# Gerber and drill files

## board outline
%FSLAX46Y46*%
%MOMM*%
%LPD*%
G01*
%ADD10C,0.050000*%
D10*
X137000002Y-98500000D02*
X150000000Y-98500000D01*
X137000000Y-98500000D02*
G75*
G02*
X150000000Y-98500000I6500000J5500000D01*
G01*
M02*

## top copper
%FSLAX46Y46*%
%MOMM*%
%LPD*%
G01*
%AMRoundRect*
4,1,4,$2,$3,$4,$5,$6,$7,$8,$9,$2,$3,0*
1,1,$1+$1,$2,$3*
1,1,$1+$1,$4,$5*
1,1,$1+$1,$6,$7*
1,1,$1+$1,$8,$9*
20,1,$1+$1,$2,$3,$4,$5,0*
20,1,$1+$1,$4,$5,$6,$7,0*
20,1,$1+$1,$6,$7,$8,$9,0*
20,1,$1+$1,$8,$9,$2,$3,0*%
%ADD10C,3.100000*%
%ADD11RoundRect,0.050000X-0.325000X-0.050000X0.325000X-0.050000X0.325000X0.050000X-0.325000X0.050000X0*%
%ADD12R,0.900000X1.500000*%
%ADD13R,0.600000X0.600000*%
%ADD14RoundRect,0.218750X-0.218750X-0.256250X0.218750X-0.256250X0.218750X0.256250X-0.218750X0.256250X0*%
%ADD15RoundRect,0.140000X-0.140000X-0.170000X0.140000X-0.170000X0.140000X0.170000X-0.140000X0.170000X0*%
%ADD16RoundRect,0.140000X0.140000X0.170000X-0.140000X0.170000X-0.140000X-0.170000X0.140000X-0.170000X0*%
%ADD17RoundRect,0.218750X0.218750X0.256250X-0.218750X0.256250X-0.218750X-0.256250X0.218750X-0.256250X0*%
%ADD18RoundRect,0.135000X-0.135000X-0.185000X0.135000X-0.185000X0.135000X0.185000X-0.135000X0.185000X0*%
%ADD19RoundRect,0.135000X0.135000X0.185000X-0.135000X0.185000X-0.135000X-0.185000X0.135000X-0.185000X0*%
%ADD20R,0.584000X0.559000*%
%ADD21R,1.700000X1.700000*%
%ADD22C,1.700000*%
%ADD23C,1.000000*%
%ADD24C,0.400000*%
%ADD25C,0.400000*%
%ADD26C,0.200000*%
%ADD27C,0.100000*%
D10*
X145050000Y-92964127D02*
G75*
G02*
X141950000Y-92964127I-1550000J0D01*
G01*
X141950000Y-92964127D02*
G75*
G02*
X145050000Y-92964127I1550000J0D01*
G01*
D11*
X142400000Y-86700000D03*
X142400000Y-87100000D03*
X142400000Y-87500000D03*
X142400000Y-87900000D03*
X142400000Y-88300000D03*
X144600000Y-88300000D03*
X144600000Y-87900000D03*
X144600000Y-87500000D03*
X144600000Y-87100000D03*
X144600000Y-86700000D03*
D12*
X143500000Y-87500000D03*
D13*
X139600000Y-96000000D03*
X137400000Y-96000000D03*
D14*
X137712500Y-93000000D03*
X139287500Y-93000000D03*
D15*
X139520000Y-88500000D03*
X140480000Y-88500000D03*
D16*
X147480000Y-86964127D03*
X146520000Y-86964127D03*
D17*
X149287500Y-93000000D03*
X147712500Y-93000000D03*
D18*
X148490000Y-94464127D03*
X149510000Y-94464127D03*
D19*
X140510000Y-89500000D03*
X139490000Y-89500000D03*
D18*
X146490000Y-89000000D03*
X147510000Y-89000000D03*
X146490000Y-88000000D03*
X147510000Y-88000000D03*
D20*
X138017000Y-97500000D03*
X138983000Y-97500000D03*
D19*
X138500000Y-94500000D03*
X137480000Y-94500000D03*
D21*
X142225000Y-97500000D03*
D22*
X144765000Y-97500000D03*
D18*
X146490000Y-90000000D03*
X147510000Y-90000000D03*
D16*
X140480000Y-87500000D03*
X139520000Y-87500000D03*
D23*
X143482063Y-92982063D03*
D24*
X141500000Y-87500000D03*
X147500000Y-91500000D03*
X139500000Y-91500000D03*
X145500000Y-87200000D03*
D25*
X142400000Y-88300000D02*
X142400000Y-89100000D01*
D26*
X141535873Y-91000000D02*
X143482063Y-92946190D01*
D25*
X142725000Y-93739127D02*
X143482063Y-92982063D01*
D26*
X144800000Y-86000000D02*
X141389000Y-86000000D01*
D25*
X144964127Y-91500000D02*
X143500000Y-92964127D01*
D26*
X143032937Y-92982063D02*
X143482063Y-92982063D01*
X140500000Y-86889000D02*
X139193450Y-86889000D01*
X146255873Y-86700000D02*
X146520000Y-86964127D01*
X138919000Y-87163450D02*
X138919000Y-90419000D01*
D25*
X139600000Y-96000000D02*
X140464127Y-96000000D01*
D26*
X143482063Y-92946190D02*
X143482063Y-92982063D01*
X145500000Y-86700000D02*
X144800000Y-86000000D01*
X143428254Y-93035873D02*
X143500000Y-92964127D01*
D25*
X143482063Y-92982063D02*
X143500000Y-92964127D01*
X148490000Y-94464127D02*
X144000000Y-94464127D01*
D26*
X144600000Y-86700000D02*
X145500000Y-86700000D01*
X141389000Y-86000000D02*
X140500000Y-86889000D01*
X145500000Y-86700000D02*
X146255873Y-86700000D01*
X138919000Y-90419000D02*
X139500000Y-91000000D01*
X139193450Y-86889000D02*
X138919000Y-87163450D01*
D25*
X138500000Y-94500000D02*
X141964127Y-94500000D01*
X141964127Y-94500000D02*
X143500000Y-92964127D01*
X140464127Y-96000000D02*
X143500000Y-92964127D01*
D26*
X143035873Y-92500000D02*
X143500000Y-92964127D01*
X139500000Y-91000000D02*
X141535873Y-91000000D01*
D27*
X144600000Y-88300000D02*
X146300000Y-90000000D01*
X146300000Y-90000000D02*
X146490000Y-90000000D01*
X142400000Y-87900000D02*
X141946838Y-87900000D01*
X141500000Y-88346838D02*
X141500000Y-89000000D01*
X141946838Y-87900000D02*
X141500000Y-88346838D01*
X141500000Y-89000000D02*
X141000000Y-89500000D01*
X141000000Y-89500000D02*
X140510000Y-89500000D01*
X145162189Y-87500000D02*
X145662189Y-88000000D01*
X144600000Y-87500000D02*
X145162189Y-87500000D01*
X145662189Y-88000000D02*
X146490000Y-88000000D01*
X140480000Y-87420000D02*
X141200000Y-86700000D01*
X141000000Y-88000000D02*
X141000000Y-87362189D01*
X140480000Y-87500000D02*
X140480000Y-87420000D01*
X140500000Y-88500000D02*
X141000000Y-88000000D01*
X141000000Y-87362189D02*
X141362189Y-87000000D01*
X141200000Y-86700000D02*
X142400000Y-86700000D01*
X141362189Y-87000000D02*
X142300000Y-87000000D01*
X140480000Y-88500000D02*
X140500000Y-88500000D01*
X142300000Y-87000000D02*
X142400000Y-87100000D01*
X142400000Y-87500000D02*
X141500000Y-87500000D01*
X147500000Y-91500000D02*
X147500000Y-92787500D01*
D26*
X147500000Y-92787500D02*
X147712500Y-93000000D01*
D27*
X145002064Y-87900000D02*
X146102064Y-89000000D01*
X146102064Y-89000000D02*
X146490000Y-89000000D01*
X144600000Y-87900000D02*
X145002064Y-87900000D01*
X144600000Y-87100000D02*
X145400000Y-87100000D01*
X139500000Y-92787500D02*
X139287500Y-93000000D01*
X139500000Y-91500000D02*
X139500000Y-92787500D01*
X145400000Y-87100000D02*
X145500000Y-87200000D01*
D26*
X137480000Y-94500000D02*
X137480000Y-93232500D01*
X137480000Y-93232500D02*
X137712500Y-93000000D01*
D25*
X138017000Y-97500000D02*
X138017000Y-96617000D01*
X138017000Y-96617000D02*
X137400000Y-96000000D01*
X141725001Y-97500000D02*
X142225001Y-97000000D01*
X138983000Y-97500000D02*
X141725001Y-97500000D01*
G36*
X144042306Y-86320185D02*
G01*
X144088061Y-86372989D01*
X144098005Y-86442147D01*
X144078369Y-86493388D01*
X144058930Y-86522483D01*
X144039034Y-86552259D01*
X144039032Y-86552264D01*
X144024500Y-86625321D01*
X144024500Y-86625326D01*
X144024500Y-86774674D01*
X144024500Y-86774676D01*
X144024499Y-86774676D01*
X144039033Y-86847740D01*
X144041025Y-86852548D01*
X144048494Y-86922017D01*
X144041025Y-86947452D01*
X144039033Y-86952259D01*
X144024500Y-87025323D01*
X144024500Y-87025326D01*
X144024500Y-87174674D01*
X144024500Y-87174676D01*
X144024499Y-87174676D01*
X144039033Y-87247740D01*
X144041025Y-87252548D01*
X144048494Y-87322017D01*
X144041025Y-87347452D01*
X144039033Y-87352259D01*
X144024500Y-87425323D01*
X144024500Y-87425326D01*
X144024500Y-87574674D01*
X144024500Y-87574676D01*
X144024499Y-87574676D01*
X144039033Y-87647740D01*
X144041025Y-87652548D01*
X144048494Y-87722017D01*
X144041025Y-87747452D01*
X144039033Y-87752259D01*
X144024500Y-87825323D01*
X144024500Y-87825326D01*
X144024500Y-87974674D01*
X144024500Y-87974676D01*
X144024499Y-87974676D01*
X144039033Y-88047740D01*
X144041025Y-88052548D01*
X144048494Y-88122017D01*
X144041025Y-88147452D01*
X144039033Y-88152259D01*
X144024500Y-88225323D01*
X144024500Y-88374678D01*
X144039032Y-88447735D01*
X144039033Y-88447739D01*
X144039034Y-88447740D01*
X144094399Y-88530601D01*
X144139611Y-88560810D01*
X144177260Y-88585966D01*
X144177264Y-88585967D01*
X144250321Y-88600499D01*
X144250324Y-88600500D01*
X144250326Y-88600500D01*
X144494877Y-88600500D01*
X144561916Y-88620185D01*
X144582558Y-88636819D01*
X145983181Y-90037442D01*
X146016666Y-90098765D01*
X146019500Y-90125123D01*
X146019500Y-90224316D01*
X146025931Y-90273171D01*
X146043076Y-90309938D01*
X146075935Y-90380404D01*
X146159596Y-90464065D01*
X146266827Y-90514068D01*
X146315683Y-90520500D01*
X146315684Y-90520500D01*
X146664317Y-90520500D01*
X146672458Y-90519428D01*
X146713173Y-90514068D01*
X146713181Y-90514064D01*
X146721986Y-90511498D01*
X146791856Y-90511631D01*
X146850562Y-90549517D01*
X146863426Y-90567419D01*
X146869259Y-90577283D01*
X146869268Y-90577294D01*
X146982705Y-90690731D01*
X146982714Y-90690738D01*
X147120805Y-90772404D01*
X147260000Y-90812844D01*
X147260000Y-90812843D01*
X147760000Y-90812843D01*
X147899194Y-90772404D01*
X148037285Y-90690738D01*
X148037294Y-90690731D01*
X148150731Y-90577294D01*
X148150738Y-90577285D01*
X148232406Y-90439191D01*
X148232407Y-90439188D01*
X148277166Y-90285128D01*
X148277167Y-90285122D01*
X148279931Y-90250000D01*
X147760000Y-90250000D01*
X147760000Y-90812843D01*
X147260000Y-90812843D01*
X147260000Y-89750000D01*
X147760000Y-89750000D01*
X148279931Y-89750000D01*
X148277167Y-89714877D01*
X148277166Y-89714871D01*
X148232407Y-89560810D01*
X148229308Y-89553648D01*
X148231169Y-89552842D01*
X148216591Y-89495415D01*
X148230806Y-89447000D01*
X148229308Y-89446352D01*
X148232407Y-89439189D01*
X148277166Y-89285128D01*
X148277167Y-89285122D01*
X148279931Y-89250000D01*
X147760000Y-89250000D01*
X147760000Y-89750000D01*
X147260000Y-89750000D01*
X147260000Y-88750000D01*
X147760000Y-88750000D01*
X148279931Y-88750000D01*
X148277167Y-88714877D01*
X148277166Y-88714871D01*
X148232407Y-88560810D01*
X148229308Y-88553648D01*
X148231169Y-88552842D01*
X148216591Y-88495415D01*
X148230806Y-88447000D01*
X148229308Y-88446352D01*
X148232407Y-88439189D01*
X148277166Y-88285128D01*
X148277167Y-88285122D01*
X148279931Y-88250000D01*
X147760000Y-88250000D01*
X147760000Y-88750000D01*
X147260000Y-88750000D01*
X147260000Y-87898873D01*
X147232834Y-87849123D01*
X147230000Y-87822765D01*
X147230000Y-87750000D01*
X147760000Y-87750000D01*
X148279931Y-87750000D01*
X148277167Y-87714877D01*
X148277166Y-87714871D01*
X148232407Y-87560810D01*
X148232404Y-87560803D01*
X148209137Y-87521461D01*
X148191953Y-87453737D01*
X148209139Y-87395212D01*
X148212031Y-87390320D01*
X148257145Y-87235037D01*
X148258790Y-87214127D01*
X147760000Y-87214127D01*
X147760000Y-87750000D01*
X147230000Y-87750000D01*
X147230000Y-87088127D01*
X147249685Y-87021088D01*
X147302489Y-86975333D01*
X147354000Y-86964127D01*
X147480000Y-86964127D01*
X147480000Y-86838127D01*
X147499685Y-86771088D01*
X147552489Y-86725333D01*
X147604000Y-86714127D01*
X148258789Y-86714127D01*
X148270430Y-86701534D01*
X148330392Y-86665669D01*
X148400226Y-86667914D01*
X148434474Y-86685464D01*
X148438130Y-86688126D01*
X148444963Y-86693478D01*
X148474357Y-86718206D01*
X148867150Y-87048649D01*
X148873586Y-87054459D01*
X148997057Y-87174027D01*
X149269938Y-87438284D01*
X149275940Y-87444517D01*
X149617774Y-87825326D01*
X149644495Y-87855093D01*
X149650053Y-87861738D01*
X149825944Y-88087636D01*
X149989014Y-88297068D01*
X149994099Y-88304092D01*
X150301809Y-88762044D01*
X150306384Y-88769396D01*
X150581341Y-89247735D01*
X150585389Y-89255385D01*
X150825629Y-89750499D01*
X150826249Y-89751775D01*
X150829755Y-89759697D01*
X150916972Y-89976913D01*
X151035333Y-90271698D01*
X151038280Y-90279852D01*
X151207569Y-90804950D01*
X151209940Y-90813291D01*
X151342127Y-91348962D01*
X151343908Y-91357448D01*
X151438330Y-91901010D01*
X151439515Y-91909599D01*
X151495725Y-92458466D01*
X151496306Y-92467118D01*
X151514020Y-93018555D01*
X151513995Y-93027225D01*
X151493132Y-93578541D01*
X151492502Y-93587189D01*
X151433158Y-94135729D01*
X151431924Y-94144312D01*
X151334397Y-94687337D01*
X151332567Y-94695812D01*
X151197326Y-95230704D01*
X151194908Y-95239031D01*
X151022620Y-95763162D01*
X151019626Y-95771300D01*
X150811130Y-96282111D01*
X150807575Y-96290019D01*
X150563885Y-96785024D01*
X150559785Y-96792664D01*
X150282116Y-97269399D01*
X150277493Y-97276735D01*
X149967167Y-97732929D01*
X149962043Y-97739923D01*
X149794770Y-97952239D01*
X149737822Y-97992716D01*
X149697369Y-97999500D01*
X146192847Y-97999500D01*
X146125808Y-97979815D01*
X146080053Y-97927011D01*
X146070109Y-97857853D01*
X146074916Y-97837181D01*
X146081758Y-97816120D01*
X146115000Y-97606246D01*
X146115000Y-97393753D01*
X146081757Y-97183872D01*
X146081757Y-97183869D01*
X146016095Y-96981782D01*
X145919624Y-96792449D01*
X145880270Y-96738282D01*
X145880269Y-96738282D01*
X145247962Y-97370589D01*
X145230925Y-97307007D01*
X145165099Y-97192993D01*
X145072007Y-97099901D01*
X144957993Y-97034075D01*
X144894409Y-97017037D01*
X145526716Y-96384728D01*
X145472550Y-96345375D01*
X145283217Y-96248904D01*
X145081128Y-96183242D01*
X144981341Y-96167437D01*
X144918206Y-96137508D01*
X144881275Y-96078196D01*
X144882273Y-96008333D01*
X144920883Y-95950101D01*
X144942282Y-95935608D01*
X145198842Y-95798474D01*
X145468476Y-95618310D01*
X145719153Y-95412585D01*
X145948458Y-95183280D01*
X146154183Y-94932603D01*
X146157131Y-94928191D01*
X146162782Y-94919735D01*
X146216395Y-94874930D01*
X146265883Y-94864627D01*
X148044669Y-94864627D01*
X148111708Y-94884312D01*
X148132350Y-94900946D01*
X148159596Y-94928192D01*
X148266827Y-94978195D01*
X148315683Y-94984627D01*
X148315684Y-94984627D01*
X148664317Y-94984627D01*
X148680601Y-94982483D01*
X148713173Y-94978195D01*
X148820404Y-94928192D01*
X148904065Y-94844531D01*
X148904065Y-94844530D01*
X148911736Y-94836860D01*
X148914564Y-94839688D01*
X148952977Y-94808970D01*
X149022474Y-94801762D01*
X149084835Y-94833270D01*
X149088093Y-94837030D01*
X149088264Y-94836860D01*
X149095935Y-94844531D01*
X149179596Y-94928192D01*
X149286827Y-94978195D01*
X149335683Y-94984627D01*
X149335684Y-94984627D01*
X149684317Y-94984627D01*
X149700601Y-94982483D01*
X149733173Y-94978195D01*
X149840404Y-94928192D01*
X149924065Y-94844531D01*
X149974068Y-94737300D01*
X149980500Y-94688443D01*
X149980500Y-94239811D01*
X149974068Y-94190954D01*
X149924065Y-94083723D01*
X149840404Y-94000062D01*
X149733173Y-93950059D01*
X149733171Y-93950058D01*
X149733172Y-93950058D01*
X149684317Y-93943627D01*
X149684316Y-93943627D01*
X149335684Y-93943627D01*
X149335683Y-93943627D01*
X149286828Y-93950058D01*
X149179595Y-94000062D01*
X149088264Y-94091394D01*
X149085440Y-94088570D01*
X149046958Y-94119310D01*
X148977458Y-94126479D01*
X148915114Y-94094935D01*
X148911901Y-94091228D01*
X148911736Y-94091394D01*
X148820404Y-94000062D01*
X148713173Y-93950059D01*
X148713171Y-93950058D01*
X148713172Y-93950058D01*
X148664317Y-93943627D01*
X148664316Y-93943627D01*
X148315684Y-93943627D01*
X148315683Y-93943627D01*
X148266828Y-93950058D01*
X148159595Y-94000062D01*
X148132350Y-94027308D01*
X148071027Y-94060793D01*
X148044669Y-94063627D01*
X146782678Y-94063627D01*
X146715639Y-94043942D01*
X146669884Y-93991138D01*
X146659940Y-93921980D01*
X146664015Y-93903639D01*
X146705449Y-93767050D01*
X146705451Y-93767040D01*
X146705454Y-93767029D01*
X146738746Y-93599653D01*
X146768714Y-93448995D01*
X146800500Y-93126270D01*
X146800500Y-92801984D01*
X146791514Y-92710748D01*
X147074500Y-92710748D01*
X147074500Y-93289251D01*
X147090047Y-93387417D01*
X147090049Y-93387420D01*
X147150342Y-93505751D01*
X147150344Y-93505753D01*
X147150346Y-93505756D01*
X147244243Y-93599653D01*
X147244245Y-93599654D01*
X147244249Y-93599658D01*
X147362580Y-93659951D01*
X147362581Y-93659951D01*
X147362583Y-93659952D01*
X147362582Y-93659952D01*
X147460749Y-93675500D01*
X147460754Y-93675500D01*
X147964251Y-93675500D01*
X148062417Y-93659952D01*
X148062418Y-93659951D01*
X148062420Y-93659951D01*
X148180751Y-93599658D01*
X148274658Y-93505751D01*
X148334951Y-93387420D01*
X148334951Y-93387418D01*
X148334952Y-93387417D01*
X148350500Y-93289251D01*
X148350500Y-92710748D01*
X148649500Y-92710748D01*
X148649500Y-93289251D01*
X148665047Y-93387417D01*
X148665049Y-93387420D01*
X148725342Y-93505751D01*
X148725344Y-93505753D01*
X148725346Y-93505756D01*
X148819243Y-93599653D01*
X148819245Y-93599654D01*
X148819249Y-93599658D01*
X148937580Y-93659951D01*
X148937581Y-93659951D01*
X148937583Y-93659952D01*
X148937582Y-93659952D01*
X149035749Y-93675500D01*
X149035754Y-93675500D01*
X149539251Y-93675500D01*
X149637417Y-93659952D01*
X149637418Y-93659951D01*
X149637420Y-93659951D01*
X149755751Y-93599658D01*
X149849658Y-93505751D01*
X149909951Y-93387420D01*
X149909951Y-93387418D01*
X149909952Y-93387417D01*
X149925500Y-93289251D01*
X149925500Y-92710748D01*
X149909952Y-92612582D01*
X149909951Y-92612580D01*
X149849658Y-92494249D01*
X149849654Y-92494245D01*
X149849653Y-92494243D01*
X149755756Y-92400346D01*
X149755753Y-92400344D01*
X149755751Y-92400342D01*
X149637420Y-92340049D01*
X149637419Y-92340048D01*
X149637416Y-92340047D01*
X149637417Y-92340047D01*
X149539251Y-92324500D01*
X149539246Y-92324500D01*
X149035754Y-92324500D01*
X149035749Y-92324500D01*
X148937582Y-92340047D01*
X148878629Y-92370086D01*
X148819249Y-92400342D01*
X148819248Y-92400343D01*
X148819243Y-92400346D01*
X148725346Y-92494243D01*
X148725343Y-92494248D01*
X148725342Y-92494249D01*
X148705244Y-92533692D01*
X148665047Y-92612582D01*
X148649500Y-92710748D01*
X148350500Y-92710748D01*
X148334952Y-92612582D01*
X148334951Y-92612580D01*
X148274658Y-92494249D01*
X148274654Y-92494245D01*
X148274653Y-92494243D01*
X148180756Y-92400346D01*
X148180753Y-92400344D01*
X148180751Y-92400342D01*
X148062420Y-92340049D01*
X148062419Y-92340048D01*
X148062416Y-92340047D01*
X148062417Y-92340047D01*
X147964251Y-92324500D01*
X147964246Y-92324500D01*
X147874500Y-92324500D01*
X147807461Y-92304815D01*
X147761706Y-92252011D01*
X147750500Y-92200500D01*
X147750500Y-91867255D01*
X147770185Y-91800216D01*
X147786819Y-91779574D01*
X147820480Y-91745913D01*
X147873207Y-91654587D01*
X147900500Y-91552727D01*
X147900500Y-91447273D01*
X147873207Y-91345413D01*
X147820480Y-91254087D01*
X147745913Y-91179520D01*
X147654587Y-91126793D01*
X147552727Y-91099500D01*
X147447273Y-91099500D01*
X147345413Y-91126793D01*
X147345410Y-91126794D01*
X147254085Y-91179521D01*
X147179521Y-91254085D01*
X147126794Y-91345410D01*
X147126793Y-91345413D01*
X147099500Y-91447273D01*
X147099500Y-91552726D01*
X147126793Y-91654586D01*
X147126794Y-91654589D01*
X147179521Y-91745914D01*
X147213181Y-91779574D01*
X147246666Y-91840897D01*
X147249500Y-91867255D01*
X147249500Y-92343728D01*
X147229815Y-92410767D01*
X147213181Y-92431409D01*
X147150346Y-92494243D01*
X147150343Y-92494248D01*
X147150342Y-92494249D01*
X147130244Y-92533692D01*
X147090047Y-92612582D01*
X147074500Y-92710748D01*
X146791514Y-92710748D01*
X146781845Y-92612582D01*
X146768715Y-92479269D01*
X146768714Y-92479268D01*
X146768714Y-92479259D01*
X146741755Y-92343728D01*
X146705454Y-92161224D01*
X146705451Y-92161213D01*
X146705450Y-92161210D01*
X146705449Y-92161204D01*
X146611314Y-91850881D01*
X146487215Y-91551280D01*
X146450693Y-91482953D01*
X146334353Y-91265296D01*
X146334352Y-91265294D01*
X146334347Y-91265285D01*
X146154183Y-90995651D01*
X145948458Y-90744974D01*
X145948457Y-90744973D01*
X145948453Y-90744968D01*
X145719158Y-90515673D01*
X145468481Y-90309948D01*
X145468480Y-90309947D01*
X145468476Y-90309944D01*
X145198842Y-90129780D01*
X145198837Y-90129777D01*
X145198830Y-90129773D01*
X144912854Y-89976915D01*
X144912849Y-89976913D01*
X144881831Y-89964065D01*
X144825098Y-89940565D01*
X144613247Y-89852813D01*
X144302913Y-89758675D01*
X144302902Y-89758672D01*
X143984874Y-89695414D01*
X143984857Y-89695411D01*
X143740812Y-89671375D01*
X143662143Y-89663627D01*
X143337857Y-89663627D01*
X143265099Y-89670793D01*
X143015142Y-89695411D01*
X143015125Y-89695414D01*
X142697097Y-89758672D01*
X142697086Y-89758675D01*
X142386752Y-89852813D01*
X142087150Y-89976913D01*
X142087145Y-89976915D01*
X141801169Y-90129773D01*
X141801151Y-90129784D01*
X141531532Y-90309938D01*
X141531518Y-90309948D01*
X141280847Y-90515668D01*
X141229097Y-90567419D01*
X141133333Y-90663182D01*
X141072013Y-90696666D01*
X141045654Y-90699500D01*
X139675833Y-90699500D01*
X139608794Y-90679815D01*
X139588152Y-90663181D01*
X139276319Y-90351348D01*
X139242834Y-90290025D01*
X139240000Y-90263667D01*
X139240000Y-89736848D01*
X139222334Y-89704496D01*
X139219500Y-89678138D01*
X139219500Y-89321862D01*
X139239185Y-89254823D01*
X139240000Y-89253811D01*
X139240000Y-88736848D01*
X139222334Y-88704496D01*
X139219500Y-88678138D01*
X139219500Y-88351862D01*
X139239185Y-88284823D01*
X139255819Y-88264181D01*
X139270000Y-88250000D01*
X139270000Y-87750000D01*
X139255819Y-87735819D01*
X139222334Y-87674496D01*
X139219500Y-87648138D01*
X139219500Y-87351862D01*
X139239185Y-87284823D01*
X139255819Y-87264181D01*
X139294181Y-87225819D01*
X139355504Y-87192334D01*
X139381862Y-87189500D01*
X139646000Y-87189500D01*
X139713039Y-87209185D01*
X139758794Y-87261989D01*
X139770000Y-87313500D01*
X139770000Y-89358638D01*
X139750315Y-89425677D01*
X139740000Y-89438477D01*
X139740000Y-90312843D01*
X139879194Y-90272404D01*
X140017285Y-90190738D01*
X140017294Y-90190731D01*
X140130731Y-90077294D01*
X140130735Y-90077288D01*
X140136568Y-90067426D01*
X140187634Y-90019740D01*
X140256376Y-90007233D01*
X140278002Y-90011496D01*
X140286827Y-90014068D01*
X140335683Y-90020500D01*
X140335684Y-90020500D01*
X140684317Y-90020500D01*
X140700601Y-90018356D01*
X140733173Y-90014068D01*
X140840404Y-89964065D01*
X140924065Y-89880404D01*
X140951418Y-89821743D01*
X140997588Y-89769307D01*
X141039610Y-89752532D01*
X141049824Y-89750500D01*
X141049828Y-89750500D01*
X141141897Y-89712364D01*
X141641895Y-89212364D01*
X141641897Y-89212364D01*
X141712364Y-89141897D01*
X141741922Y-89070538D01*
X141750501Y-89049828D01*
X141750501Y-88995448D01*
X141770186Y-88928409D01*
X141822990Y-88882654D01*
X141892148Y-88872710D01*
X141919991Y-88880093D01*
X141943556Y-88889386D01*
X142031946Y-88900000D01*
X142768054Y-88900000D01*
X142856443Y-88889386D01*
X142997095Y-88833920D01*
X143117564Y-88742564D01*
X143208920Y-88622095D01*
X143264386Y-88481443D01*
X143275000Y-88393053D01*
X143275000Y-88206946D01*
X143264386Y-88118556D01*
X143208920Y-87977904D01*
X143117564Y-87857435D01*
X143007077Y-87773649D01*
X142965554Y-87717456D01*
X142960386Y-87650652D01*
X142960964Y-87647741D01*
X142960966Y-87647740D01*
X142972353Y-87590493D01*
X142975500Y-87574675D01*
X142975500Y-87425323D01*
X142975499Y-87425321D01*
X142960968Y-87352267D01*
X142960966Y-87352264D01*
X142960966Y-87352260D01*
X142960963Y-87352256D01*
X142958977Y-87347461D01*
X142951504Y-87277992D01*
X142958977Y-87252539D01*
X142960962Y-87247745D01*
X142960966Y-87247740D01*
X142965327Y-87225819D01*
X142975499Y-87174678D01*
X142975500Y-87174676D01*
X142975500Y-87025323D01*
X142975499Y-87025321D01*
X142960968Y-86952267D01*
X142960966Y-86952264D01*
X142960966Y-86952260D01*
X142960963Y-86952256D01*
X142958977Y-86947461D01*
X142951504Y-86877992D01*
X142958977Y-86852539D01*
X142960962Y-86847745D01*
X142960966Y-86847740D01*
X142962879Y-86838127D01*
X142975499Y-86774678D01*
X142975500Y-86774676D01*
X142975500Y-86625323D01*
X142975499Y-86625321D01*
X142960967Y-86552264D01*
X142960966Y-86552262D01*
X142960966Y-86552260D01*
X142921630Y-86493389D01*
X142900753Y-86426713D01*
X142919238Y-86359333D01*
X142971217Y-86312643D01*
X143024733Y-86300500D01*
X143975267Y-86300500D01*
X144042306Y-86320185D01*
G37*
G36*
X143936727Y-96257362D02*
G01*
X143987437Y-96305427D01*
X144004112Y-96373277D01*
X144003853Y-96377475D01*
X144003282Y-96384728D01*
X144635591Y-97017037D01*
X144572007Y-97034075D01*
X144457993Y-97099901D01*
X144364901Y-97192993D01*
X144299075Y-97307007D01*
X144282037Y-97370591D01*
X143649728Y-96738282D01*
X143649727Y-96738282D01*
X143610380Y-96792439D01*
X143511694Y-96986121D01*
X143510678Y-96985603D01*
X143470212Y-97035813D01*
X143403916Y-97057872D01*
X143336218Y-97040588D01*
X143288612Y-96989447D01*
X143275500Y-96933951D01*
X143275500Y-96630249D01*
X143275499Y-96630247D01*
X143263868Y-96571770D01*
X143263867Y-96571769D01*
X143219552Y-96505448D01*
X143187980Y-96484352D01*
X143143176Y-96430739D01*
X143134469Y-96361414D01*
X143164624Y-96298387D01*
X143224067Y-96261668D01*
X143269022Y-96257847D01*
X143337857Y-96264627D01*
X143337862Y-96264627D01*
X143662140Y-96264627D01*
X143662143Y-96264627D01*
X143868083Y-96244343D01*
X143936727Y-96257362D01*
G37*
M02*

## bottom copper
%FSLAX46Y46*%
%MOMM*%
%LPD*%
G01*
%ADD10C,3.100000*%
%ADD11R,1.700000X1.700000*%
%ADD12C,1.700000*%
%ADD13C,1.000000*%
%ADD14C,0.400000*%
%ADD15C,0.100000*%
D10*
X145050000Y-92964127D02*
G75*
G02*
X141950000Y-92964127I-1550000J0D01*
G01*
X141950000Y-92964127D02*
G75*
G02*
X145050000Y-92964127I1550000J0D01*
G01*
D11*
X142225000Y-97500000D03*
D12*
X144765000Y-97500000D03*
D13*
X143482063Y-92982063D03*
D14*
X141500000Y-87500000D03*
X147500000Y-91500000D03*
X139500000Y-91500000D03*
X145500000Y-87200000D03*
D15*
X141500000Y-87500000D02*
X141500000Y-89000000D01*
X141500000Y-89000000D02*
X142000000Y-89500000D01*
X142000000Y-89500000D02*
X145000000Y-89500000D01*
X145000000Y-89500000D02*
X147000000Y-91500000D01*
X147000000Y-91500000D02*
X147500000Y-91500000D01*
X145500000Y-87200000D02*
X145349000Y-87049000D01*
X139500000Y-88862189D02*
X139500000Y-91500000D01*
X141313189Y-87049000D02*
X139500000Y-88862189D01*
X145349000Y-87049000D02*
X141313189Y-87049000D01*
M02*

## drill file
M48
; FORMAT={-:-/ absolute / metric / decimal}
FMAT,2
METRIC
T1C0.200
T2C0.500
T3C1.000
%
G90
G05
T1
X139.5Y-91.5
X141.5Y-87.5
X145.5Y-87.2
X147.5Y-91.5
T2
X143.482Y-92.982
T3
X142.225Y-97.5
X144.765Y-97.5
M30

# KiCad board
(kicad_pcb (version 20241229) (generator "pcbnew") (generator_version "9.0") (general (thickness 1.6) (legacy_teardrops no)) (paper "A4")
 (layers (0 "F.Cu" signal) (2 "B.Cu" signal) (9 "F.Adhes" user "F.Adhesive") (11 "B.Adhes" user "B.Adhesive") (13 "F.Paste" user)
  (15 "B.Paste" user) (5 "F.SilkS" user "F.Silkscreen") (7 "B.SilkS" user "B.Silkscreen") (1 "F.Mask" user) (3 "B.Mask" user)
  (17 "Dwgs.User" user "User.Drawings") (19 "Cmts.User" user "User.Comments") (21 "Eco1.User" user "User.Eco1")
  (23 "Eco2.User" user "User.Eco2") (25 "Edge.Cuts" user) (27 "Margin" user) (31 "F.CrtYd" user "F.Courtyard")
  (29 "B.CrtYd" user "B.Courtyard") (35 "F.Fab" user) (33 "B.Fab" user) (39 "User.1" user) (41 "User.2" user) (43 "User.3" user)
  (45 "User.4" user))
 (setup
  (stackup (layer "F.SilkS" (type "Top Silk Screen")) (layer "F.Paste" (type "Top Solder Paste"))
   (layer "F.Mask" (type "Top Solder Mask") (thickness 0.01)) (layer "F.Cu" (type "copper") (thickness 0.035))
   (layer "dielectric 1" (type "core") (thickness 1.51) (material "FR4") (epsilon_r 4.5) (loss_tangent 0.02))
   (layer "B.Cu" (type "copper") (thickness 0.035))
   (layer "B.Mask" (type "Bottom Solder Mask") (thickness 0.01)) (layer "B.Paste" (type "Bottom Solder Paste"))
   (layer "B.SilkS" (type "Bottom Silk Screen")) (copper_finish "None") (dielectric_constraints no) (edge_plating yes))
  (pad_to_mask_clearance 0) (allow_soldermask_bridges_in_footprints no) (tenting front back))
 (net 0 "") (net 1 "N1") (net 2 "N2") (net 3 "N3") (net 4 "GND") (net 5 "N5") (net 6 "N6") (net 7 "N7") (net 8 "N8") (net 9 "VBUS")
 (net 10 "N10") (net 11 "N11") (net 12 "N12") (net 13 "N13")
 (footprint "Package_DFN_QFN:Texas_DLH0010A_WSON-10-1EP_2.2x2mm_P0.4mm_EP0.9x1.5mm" (layer "F.Cu") (at 143.5 87.5)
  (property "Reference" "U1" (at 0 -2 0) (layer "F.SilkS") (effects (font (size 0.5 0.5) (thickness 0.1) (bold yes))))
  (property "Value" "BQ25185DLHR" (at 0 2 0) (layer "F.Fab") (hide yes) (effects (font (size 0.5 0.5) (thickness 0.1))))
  (pad "" smd roundrect (at 0 0) (size 0.84 1.41) (layers "F.Paste") (roundrect_rratio 0.25))
  (pad "1" smd roundrect (at -1.1 -0.8) (size 0.75 0.2) (layers "F.Cu" "F.Mask" "F.Paste") (roundrect_rratio 0.25) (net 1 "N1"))
  (pad "2" smd roundrect (at -1.1 -0.4) (size 0.75 0.2) (layers "F.Cu" "F.Mask" "F.Paste") (roundrect_rratio 0.25) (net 1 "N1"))
  (pad "3" smd roundrect (at -1.1 0) (size 0.75 0.2) (layers "F.Cu" "F.Mask" "F.Paste") (roundrect_rratio 0.25) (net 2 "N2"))
  (pad "4" smd roundrect (at -1.1 0.4) (size 0.75 0.2) (layers "F.Cu" "F.Mask" "F.Paste") (roundrect_rratio 0.25) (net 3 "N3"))
  (pad "5" smd roundrect (at -1.1 0.8) (size 0.75 0.2) (layers "F.Cu" "F.Mask" "F.Paste") (roundrect_rratio 0.25) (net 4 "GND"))
  (pad "6" smd roundrect (at 1.1 0.8) (size 0.75 0.2) (layers "F.Cu" "F.Mask" "F.Paste") (roundrect_rratio 0.25) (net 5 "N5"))
  (pad "7" smd roundrect (at 1.1 0.4) (size 0.75 0.2) (layers "F.Cu" "F.Mask" "F.Paste") (roundrect_rratio 0.25) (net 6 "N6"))
  (pad "8" smd roundrect (at 1.1 0) (size 0.75 0.2) (layers "F.Cu" "F.Mask" "F.Paste") (roundrect_rratio 0.25) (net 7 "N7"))
  (pad "9" smd roundrect (at 1.1 -0.4) (size 0.75 0.2) (layers "F.Cu" "F.Mask" "F.Paste") (roundrect_rratio 0.25) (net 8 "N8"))
  (pad "10" smd roundrect (at 1.1 -0.8) (size 0.75 0.2) (layers "F.Cu" "F.Mask" "F.Paste") (roundrect_rratio 0.25) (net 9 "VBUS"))
  (pad "11" smd rect (at 0 0) (size 0.9 1.5) (layers "F.Cu" "F.Mask") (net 4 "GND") (zone_connect 2)))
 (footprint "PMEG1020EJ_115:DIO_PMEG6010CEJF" (layer "F.Cu") (at 138.5 96 180)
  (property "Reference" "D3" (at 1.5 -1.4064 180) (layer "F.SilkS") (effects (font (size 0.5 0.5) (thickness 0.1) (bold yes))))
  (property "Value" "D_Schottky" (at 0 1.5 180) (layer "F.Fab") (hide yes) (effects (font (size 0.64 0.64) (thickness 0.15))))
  (pad "1" smd rect (at -1.1 0 180) (size 0.6 0.6) (layers "F.Cu" "F.Mask") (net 9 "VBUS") (solder_mask_margin 0.102))
  (pad "2" smd rect (at 1.1 0 180) (size 0.6 0.6) (layers "F.Cu" "F.Mask") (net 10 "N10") (solder_mask_margin 0.102)))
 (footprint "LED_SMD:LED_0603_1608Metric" (layer "F.Cu") (at 138.5 93)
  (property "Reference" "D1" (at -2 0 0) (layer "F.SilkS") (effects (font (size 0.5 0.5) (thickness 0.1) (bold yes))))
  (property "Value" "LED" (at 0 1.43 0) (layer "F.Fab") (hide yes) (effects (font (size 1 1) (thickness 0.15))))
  (pad "1" smd roundrect (at -0.7875 0) (size 0.875 0.95) (layers "F.Cu" "F.Mask" "F.Paste") (roundrect_rratio 0.25) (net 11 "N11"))
  (pad "2" smd roundrect (at 0.7875 0) (size 0.875 0.95) (layers "F.Cu" "F.Mask" "F.Paste") (roundrect_rratio 0.25) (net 8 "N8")))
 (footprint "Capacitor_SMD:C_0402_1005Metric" (layer "F.Cu") (at 140 88.5)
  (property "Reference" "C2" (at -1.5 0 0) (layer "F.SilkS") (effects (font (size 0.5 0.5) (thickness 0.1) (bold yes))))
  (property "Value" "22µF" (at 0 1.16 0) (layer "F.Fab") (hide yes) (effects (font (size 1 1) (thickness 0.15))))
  (pad "1" smd roundrect (at -0.48 0) (size 0.56 0.62) (layers "F.Cu" "F.Mask" "F.Paste") (roundrect_rratio 0.25) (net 4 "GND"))
  (pad "2" smd roundrect (at 0.48 0) (size 0.56 0.62) (layers "F.Cu" "F.Mask" "F.Paste") (roundrect_rratio 0.25) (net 1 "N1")))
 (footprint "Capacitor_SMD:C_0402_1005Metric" (layer "F.Cu") (at 147 86.964127 180)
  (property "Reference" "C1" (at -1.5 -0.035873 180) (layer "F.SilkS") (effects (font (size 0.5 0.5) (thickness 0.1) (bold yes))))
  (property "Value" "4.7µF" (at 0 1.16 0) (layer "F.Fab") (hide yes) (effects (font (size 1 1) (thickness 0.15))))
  (pad "1" smd roundrect (at -0.48 0 180) (size 0.56 0.62) (layers "F.Cu" "F.Mask" "F.Paste") (roundrect_rratio 0.25) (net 4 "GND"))
  (pad "2" smd roundrect (at 0.48 0 180) (size 0.56 0.62) (layers "F.Cu" "F.Mask" "F.Paste") (roundrect_rratio 0.25) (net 9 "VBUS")))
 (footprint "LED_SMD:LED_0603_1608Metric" (layer "F.Cu") (at 148.5 93 180)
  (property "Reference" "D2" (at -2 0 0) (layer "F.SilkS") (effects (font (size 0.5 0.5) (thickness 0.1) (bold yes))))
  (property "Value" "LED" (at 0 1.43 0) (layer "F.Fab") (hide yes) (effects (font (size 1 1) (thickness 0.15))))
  (pad "1" smd roundrect (at -0.7875 0 180) (size 0.875 0.95) (layers "F.Cu" "F.Mask" "F.Paste") (roundrect_rratio 0.25) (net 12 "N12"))
  (pad "2" smd roundrect (at 0.7875 0 180) (size 0.875 0.95) (layers "F.Cu" "F.Mask" "F.Paste") (roundrect_rratio 0.25) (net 2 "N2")))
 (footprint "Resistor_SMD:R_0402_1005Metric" (layer "F.Cu") (at 149 94.464127)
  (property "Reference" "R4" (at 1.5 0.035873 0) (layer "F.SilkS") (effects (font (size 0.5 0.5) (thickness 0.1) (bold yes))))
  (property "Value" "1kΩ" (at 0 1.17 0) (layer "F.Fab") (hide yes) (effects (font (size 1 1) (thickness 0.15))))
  (pad "1" smd roundrect (at -0.51 0) (size 0.54 0.64) (layers "F.Cu" "F.Mask" "F.Paste") (roundrect_rratio 0.25) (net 9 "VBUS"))
  (pad "2" smd roundrect (at 0.51 0) (size 0.54 0.64) (layers "F.Cu" "F.Mask" "F.Paste") (roundrect_rratio 0.25) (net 12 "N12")))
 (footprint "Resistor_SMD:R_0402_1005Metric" (layer "F.Cu") (at 140 89.5 180)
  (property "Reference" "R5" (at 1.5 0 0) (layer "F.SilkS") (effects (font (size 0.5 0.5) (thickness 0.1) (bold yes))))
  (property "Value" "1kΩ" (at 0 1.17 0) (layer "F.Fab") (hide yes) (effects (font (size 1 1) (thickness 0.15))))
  (pad "1" smd roundrect (at -0.51 0 180) (size 0.54 0.64) (layers "F.Cu" "F.Mask" "F.Paste") (roundrect_rratio 0.25) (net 3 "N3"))
  (pad "2" smd roundrect (at 0.51 0 180) (size 0.54 0.64) (layers "F.Cu" "F.Mask" "F.Paste") (roundrect_rratio 0.25) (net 4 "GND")))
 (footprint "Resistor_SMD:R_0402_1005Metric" (layer "F.Cu") (at 147 89)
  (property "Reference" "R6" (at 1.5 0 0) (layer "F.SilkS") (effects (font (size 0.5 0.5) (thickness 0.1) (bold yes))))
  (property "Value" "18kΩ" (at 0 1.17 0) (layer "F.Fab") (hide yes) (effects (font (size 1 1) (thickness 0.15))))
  (pad "1" smd roundrect (at -0.51 0) (size 0.54 0.64) (layers "F.Cu" "F.Mask" "F.Paste") (roundrect_rratio 0.25) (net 6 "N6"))
  (pad "2" smd roundrect (at 0.51 0) (size 0.54 0.64) (layers "F.Cu" "F.Mask" "F.Paste") (roundrect_rratio 0.25) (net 4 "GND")))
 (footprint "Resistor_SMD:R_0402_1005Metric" (layer "F.Cu") (at 147 88)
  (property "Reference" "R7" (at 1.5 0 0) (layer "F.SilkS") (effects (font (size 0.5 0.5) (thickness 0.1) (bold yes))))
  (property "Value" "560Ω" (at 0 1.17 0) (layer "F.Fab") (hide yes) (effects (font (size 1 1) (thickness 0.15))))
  (pad "1" smd roundrect (at -0.51 0) (size 0.54 0.64) (layers "F.Cu" "F.Mask" "F.Paste") (roundrect_rratio 0.25) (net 7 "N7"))
  (pad "2" smd roundrect (at 0.51 0) (size 0.54 0.64) (layers "F.Cu" "F.Mask" "F.Paste") (roundrect_rratio 0.25) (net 4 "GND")))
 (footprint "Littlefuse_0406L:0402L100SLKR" (layer "F.Cu") (at 138.5 97.5)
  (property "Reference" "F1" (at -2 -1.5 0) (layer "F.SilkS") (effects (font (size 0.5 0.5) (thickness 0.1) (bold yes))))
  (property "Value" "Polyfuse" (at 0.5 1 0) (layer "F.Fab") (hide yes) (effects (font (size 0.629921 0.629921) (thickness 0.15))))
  (pad "1" smd rect (at -0.483 0) (size 0.584 0.559) (layers "F.Cu" "F.Mask" "F.Paste") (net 10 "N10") (solder_mask_margin 0.102))
  (pad "2" smd rect (at 0.483 0) (size 0.584 0.559) (layers "F.Cu" "F.Mask" "F.Paste") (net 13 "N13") (solder_mask_margin 0.102)))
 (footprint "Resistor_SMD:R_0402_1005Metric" (layer "F.Cu") (at 137.99 94.5 180)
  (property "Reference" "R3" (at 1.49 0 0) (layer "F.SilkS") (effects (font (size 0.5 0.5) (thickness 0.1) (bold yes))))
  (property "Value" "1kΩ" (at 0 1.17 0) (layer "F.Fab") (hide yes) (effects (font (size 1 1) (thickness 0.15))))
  (pad "1" smd roundrect (at -0.51 0 180) (size 0.54 0.64) (layers "F.Cu" "F.Mask" "F.Paste") (roundrect_rratio 0.25) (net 9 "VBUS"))
  (pad "2" smd roundrect (at 0.51 0 180) (size 0.54 0.64) (layers "F.Cu" "F.Mask" "F.Paste") (roundrect_rratio 0.25) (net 11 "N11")))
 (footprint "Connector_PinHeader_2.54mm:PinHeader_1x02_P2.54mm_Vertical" (layer "F.Cu") (at 142.225 97.5 90)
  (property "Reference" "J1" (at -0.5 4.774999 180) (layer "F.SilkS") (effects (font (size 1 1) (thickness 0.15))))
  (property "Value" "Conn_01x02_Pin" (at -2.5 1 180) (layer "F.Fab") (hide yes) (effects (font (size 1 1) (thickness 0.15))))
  (pad "1" thru_hole rect (at 0 0 90) (size 1.7 1.7) (drill 1) (layers "*.Cu" "*.Mask") (remove_unused_layers no) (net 13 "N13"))
  (pad "2" thru_hole circle (at 0 2.54 90) (size 1.7 1.7) (drill 1) (layers "*.Cu" "*.Mask") (remove_unused_layers no) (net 4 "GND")))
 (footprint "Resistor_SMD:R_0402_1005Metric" (layer "F.Cu") (at 147 90)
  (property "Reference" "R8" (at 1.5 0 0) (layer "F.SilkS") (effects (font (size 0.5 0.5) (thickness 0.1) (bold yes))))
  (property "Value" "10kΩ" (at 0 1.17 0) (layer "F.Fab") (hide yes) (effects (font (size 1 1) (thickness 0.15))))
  (pad "1" smd roundrect (at -0.51 0) (size 0.54 0.64) (layers "F.Cu" "F.Mask" "F.Paste") (roundrect_rratio 0.25) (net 5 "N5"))
  (pad "2" smd roundrect (at 0.51 0) (size 0.54 0.64) (layers "F.Cu" "F.Mask" "F.Paste") (roundrect_rratio 0.25) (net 4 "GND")))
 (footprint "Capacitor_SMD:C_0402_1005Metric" (layer "F.Cu") (at 140 87.5 180)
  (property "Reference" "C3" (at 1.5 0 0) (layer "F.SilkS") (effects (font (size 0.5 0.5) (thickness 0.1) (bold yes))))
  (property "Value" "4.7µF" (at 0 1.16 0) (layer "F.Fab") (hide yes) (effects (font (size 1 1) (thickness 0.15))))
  (pad "1" smd roundrect (at -0.48 0 180) (size 0.56 0.62) (layers "F.Cu" "F.Mask" "F.Paste") (roundrect_rratio 0.25) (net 1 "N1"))
  (pad "2" smd roundrect (at 0.48 0 180) (size 0.56 0.62) (layers "F.Cu" "F.Mask" "F.Paste") (roundrect_rratio 0.25) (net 4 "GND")))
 (gr_circle (center 143.5 92.964127) (end 146.5 92.964127) (stroke (width 0.2) (type solid)) (fill yes) (layer "F.Cu") (net 9))
 (gr_circle (center 143.5 92.964127) (end 146.5 92.964127) (stroke (width 0.2) (type solid)) (fill yes) (layer "B.Cu") (net 9))
 (gr_line (start 137.000002 98.5) (end 150 98.5) (stroke (width 0.05) (type default)) (layer "Edge.Cuts"))
 (gr_arc (start 137 98.5) (mid 143.5 84.485307) (end 150 98.5) (stroke (width 0.05) (type default)) (layer "Edge.Cuts"))
 (segment (start 142.4 88.3) (end 142.4 89.1) (width 0.4) (layer "F.Cu") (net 4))
 (segment (start 141.535873 91) (end 143.482063 92.94619) (width 0.2) (layer "F.Cu") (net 9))
 (segment (start 142.725 93.739127) (end 143.482063 92.982063) (width 0.4) (layer "F.Cu") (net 9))
 (segment (start 144.8 86) (end 141.389 86) (width 0.2) (layer "F.Cu") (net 9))
 (segment (start 144.964127 91.5) (end 143.5 92.964127) (width 0.4) (layer "F.Cu") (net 9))
 (segment (start 143.032937 92.982063) (end 143.482063 92.982063) (width 0.2) (layer "F.Cu") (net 9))
 (segment (start 140.5 86.889) (end 139.19345 86.889) (width 0.2) (layer "F.Cu") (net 9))
 (segment (start 146.255873 86.7) (end 146.52 86.964127) (width 0.2) (layer "F.Cu") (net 9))
 (segment (start 138.919 87.16345) (end 138.919 90.419) (width 0.2) (layer "F.Cu") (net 9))
 (segment (start 139.6 96) (end 140.464127 96) (width 0.4) (layer "F.Cu") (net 9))
 (segment (start 143.482063 92.94619) (end 143.482063 92.982063) (width 0.2) (layer "F.Cu") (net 9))
 (segment (start 145.5 86.7) (end 144.8 86) (width 0.2) (layer "F.Cu") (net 9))
 (segment (start 143.428254 93.035873) (end 143.5 92.964127) (width 0.2) (layer "F.Cu") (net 9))
 (segment (start 143.482063 92.982063) (end 143.5 92.964127) (width 0.4) (layer "F.Cu") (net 9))
 (segment (start 148.49 94.464127) (end 144 94.464127) (width 0.4) (layer "F.Cu") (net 9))
 (segment (start 144.6 86.7) (end 145.5 86.7) (width 0.2) (layer "F.Cu") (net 9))
 (segment (start 141.389 86) (end 140.5 86.889) (width 0.2) (layer "F.Cu") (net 9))
 (segment (start 145.5 86.7) (end 146.255873 86.7) (width 0.2) (layer "F.Cu") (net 9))
 (segment (start 138.919 90.419) (end 139.5 91) (width 0.2) (layer "F.Cu") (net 9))
 (segment (start 139.19345 86.889) (end 138.919 87.16345) (width 0.2) (layer "F.Cu") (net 9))
 (segment (start 138.5 94.5) (end 141.964127 94.5) (width 0.4) (layer "F.Cu") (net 9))
 (segment (start 141.964127 94.5) (end 143.5 92.964127) (width 0.4) (layer "F.Cu") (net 9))
 (segment (start 140.464127 96) (end 143.5 92.964127) (width 0.4) (layer "F.Cu") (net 9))
 (segment (start 143.035873 92.5) (end 143.5 92.964127) (width 0.2) (layer "F.Cu") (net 9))
 (segment (start 139.5 91) (end 141.535873 91) (width 0.2) (layer "F.Cu") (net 9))
 (via (at 143.482063 92.982063) (size 1) (drill 0.5) (layers "F.Cu" "B.Cu") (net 9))
 (segment (start 144.6 88.3) (end 146.3 90) (width 0.1) (layer "F.Cu") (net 5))
 (segment (start 146.3 90) (end 146.49 90) (width 0.1) (layer "F.Cu") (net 5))
 (segment (start 142.4 87.9) (end 141.946838 87.9) (width 0.1) (layer "F.Cu") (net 3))
 (segment (start 141.5 88.346838) (end 141.5 89) (width 0.1) (layer "F.Cu") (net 3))
 (segment (start 141.946838 87.9) (end 141.5 88.346838) (width 0.1) (layer "F.Cu") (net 3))
 (segment (start 141.5 89) (end 141 89.5) (width 0.1) (layer "F.Cu") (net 3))
 (segment (start 141 89.5) (end 140.51 89.5) (width 0.1) (layer "F.Cu") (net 3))
 (segment (start 145.162189 87.5) (end 145.662189 88) (width 0.1) (layer "F.Cu") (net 7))
 (segment (start 144.6 87.5) (end 145.162189 87.5) (width 0.1) (layer "F.Cu") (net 7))
 (segment (start 145.662189 88) (end 146.49 88) (width 0.1) (layer "F.Cu") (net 7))
 (segment (start 140.48 87.42) (end 141.2 86.7) (width 0.1) (layer "F.Cu") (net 1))
 (segment (start 141 88) (end 141 87.362189) (width 0.1) (layer "F.Cu") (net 1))
 (segment (start 140.48 87.5) (end 140.48 87.42) (width 0.1) (layer "F.Cu") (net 1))
 (segment (start 140.5 88.5) (end 141 88) (width 0.1) (layer "F.Cu") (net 1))
 (segment (start 141 87.362189) (end 141.362189 87) (width 0.1) (layer "F.Cu") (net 1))
 (segment (start 141.2 86.7) (end 142.4 86.7) (width 0.1) (layer "F.Cu") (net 1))
 (segment (start 141.362189 87) (end 142.3 87) (width 0.1) (layer "F.Cu") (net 1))
 (segment (start 140.48 88.5) (end 140.5 88.5) (width 0.1) (layer "F.Cu") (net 1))
 (segment (start 142.3 87) (end 142.4 87.1) (width 0.1) (layer "F.Cu") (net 1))
 (segment (start 142.4 87.5) (end 141.5 87.5) (width 0.1) (layer "F.Cu") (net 2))
 (segment (start 147.5 91.5) (end 147.5 92.7875) (width 0.1) (layer "F.Cu") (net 2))
 (segment (start 147.5 92.7875) (end 147.7125 93) (width 0.2) (layer "F.Cu") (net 2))
 (via (at 141.5 87.5) (size 0.4) (drill 0.2) (layers "F.Cu" "B.Cu") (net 2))
 (via (at 147.5 91.5) (size 0.4) (drill 0.2) (layers "F.Cu" "B.Cu") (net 2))
 (segment (start 141.5 87.5) (end 141.5 89) (width 0.1) (layer "B.Cu") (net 2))
 (segment (start 141.5 89) (end 142 89.5) (width 0.1) (layer "B.Cu") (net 2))
 (segment (start 142 89.5) (end 145 89.5) (width 0.1) (layer "B.Cu") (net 2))
 (segment (start 145 89.5) (end 147 91.5) (width 0.1) (layer "B.Cu") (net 2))
 (segment (start 147 91.5) (end 147.5 91.5) (width 0.1) (layer "B.Cu") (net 2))
 (segment (start 145.002064 87.9) (end 146.102064 89) (width 0.1) (layer "F.Cu") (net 6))
 (segment (start 146.102064 89) (end 146.49 89) (width 0.1) (layer "F.Cu") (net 6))
 (segment (start 144.6 87.9) (end 145.002064 87.9) (width 0.1) (layer "F.Cu") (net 6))
 (segment (start 144.6 87.1) (end 145.4 87.1) (width 0.1) (layer "F.Cu") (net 8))
 (segment (start 139.5 92.7875) (end 139.2875 93) (width 0.1) (layer "F.Cu") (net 8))
 (segment (start 139.5 91.5) (end 139.5 92.7875) (width 0.1) (layer "F.Cu") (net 8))
 (segment (start 145.4 87.1) (end 145.5 87.2) (width 0.1) (layer "F.Cu") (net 8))
 (via (at 139.5 91.5) (size 0.4) (drill 0.2) (layers "F.Cu" "B.Cu") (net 8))
 (via (at 145.5 87.2) (size 0.4) (drill 0.2) (layers "F.Cu" "B.Cu") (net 8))
 (segment (start 145.5 87.2) (end 145.349 87.049) (width 0.1) (layer "B.Cu") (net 8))
 (segment (start 139.5 88.862189) (end 139.5 91.5) (width 0.1) (layer "B.Cu") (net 8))
 (segment (start 141.313189 87.049) (end 139.5 88.862189) (width 0.1) (layer "B.Cu") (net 8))
 (segment (start 145.349 87.049) (end 141.313189 87.049) (width 0.1) (layer "B.Cu") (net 8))
 (segment (start 137.48 94.5) (end 137.48 93.2325) (width 0.2) (layer "F.Cu") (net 11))
 (segment (start 137.48 93.2325) (end 137.7125 93) (width 0.2) (layer "F.Cu") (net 11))
 (segment (start 138.017 97.5) (end 138.017 96.617) (width 0.4) (layer "F.Cu") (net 10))
 (segment (start 138.017 96.617) (end 137.4 96) (width 0.4) (layer "F.Cu") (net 10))
 (segment (start 141.725001 97.5) (end 142.225001 97) (width 0.4) (layer "F.Cu") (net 13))
 (segment (start 138.983 97.5) (end 141.725001 97.5) (width 0.4) (layer "F.Cu") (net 13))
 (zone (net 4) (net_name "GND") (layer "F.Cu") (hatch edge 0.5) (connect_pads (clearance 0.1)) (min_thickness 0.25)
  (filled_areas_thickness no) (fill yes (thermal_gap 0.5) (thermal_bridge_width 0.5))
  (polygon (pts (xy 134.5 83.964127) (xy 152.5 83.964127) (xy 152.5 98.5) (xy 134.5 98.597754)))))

